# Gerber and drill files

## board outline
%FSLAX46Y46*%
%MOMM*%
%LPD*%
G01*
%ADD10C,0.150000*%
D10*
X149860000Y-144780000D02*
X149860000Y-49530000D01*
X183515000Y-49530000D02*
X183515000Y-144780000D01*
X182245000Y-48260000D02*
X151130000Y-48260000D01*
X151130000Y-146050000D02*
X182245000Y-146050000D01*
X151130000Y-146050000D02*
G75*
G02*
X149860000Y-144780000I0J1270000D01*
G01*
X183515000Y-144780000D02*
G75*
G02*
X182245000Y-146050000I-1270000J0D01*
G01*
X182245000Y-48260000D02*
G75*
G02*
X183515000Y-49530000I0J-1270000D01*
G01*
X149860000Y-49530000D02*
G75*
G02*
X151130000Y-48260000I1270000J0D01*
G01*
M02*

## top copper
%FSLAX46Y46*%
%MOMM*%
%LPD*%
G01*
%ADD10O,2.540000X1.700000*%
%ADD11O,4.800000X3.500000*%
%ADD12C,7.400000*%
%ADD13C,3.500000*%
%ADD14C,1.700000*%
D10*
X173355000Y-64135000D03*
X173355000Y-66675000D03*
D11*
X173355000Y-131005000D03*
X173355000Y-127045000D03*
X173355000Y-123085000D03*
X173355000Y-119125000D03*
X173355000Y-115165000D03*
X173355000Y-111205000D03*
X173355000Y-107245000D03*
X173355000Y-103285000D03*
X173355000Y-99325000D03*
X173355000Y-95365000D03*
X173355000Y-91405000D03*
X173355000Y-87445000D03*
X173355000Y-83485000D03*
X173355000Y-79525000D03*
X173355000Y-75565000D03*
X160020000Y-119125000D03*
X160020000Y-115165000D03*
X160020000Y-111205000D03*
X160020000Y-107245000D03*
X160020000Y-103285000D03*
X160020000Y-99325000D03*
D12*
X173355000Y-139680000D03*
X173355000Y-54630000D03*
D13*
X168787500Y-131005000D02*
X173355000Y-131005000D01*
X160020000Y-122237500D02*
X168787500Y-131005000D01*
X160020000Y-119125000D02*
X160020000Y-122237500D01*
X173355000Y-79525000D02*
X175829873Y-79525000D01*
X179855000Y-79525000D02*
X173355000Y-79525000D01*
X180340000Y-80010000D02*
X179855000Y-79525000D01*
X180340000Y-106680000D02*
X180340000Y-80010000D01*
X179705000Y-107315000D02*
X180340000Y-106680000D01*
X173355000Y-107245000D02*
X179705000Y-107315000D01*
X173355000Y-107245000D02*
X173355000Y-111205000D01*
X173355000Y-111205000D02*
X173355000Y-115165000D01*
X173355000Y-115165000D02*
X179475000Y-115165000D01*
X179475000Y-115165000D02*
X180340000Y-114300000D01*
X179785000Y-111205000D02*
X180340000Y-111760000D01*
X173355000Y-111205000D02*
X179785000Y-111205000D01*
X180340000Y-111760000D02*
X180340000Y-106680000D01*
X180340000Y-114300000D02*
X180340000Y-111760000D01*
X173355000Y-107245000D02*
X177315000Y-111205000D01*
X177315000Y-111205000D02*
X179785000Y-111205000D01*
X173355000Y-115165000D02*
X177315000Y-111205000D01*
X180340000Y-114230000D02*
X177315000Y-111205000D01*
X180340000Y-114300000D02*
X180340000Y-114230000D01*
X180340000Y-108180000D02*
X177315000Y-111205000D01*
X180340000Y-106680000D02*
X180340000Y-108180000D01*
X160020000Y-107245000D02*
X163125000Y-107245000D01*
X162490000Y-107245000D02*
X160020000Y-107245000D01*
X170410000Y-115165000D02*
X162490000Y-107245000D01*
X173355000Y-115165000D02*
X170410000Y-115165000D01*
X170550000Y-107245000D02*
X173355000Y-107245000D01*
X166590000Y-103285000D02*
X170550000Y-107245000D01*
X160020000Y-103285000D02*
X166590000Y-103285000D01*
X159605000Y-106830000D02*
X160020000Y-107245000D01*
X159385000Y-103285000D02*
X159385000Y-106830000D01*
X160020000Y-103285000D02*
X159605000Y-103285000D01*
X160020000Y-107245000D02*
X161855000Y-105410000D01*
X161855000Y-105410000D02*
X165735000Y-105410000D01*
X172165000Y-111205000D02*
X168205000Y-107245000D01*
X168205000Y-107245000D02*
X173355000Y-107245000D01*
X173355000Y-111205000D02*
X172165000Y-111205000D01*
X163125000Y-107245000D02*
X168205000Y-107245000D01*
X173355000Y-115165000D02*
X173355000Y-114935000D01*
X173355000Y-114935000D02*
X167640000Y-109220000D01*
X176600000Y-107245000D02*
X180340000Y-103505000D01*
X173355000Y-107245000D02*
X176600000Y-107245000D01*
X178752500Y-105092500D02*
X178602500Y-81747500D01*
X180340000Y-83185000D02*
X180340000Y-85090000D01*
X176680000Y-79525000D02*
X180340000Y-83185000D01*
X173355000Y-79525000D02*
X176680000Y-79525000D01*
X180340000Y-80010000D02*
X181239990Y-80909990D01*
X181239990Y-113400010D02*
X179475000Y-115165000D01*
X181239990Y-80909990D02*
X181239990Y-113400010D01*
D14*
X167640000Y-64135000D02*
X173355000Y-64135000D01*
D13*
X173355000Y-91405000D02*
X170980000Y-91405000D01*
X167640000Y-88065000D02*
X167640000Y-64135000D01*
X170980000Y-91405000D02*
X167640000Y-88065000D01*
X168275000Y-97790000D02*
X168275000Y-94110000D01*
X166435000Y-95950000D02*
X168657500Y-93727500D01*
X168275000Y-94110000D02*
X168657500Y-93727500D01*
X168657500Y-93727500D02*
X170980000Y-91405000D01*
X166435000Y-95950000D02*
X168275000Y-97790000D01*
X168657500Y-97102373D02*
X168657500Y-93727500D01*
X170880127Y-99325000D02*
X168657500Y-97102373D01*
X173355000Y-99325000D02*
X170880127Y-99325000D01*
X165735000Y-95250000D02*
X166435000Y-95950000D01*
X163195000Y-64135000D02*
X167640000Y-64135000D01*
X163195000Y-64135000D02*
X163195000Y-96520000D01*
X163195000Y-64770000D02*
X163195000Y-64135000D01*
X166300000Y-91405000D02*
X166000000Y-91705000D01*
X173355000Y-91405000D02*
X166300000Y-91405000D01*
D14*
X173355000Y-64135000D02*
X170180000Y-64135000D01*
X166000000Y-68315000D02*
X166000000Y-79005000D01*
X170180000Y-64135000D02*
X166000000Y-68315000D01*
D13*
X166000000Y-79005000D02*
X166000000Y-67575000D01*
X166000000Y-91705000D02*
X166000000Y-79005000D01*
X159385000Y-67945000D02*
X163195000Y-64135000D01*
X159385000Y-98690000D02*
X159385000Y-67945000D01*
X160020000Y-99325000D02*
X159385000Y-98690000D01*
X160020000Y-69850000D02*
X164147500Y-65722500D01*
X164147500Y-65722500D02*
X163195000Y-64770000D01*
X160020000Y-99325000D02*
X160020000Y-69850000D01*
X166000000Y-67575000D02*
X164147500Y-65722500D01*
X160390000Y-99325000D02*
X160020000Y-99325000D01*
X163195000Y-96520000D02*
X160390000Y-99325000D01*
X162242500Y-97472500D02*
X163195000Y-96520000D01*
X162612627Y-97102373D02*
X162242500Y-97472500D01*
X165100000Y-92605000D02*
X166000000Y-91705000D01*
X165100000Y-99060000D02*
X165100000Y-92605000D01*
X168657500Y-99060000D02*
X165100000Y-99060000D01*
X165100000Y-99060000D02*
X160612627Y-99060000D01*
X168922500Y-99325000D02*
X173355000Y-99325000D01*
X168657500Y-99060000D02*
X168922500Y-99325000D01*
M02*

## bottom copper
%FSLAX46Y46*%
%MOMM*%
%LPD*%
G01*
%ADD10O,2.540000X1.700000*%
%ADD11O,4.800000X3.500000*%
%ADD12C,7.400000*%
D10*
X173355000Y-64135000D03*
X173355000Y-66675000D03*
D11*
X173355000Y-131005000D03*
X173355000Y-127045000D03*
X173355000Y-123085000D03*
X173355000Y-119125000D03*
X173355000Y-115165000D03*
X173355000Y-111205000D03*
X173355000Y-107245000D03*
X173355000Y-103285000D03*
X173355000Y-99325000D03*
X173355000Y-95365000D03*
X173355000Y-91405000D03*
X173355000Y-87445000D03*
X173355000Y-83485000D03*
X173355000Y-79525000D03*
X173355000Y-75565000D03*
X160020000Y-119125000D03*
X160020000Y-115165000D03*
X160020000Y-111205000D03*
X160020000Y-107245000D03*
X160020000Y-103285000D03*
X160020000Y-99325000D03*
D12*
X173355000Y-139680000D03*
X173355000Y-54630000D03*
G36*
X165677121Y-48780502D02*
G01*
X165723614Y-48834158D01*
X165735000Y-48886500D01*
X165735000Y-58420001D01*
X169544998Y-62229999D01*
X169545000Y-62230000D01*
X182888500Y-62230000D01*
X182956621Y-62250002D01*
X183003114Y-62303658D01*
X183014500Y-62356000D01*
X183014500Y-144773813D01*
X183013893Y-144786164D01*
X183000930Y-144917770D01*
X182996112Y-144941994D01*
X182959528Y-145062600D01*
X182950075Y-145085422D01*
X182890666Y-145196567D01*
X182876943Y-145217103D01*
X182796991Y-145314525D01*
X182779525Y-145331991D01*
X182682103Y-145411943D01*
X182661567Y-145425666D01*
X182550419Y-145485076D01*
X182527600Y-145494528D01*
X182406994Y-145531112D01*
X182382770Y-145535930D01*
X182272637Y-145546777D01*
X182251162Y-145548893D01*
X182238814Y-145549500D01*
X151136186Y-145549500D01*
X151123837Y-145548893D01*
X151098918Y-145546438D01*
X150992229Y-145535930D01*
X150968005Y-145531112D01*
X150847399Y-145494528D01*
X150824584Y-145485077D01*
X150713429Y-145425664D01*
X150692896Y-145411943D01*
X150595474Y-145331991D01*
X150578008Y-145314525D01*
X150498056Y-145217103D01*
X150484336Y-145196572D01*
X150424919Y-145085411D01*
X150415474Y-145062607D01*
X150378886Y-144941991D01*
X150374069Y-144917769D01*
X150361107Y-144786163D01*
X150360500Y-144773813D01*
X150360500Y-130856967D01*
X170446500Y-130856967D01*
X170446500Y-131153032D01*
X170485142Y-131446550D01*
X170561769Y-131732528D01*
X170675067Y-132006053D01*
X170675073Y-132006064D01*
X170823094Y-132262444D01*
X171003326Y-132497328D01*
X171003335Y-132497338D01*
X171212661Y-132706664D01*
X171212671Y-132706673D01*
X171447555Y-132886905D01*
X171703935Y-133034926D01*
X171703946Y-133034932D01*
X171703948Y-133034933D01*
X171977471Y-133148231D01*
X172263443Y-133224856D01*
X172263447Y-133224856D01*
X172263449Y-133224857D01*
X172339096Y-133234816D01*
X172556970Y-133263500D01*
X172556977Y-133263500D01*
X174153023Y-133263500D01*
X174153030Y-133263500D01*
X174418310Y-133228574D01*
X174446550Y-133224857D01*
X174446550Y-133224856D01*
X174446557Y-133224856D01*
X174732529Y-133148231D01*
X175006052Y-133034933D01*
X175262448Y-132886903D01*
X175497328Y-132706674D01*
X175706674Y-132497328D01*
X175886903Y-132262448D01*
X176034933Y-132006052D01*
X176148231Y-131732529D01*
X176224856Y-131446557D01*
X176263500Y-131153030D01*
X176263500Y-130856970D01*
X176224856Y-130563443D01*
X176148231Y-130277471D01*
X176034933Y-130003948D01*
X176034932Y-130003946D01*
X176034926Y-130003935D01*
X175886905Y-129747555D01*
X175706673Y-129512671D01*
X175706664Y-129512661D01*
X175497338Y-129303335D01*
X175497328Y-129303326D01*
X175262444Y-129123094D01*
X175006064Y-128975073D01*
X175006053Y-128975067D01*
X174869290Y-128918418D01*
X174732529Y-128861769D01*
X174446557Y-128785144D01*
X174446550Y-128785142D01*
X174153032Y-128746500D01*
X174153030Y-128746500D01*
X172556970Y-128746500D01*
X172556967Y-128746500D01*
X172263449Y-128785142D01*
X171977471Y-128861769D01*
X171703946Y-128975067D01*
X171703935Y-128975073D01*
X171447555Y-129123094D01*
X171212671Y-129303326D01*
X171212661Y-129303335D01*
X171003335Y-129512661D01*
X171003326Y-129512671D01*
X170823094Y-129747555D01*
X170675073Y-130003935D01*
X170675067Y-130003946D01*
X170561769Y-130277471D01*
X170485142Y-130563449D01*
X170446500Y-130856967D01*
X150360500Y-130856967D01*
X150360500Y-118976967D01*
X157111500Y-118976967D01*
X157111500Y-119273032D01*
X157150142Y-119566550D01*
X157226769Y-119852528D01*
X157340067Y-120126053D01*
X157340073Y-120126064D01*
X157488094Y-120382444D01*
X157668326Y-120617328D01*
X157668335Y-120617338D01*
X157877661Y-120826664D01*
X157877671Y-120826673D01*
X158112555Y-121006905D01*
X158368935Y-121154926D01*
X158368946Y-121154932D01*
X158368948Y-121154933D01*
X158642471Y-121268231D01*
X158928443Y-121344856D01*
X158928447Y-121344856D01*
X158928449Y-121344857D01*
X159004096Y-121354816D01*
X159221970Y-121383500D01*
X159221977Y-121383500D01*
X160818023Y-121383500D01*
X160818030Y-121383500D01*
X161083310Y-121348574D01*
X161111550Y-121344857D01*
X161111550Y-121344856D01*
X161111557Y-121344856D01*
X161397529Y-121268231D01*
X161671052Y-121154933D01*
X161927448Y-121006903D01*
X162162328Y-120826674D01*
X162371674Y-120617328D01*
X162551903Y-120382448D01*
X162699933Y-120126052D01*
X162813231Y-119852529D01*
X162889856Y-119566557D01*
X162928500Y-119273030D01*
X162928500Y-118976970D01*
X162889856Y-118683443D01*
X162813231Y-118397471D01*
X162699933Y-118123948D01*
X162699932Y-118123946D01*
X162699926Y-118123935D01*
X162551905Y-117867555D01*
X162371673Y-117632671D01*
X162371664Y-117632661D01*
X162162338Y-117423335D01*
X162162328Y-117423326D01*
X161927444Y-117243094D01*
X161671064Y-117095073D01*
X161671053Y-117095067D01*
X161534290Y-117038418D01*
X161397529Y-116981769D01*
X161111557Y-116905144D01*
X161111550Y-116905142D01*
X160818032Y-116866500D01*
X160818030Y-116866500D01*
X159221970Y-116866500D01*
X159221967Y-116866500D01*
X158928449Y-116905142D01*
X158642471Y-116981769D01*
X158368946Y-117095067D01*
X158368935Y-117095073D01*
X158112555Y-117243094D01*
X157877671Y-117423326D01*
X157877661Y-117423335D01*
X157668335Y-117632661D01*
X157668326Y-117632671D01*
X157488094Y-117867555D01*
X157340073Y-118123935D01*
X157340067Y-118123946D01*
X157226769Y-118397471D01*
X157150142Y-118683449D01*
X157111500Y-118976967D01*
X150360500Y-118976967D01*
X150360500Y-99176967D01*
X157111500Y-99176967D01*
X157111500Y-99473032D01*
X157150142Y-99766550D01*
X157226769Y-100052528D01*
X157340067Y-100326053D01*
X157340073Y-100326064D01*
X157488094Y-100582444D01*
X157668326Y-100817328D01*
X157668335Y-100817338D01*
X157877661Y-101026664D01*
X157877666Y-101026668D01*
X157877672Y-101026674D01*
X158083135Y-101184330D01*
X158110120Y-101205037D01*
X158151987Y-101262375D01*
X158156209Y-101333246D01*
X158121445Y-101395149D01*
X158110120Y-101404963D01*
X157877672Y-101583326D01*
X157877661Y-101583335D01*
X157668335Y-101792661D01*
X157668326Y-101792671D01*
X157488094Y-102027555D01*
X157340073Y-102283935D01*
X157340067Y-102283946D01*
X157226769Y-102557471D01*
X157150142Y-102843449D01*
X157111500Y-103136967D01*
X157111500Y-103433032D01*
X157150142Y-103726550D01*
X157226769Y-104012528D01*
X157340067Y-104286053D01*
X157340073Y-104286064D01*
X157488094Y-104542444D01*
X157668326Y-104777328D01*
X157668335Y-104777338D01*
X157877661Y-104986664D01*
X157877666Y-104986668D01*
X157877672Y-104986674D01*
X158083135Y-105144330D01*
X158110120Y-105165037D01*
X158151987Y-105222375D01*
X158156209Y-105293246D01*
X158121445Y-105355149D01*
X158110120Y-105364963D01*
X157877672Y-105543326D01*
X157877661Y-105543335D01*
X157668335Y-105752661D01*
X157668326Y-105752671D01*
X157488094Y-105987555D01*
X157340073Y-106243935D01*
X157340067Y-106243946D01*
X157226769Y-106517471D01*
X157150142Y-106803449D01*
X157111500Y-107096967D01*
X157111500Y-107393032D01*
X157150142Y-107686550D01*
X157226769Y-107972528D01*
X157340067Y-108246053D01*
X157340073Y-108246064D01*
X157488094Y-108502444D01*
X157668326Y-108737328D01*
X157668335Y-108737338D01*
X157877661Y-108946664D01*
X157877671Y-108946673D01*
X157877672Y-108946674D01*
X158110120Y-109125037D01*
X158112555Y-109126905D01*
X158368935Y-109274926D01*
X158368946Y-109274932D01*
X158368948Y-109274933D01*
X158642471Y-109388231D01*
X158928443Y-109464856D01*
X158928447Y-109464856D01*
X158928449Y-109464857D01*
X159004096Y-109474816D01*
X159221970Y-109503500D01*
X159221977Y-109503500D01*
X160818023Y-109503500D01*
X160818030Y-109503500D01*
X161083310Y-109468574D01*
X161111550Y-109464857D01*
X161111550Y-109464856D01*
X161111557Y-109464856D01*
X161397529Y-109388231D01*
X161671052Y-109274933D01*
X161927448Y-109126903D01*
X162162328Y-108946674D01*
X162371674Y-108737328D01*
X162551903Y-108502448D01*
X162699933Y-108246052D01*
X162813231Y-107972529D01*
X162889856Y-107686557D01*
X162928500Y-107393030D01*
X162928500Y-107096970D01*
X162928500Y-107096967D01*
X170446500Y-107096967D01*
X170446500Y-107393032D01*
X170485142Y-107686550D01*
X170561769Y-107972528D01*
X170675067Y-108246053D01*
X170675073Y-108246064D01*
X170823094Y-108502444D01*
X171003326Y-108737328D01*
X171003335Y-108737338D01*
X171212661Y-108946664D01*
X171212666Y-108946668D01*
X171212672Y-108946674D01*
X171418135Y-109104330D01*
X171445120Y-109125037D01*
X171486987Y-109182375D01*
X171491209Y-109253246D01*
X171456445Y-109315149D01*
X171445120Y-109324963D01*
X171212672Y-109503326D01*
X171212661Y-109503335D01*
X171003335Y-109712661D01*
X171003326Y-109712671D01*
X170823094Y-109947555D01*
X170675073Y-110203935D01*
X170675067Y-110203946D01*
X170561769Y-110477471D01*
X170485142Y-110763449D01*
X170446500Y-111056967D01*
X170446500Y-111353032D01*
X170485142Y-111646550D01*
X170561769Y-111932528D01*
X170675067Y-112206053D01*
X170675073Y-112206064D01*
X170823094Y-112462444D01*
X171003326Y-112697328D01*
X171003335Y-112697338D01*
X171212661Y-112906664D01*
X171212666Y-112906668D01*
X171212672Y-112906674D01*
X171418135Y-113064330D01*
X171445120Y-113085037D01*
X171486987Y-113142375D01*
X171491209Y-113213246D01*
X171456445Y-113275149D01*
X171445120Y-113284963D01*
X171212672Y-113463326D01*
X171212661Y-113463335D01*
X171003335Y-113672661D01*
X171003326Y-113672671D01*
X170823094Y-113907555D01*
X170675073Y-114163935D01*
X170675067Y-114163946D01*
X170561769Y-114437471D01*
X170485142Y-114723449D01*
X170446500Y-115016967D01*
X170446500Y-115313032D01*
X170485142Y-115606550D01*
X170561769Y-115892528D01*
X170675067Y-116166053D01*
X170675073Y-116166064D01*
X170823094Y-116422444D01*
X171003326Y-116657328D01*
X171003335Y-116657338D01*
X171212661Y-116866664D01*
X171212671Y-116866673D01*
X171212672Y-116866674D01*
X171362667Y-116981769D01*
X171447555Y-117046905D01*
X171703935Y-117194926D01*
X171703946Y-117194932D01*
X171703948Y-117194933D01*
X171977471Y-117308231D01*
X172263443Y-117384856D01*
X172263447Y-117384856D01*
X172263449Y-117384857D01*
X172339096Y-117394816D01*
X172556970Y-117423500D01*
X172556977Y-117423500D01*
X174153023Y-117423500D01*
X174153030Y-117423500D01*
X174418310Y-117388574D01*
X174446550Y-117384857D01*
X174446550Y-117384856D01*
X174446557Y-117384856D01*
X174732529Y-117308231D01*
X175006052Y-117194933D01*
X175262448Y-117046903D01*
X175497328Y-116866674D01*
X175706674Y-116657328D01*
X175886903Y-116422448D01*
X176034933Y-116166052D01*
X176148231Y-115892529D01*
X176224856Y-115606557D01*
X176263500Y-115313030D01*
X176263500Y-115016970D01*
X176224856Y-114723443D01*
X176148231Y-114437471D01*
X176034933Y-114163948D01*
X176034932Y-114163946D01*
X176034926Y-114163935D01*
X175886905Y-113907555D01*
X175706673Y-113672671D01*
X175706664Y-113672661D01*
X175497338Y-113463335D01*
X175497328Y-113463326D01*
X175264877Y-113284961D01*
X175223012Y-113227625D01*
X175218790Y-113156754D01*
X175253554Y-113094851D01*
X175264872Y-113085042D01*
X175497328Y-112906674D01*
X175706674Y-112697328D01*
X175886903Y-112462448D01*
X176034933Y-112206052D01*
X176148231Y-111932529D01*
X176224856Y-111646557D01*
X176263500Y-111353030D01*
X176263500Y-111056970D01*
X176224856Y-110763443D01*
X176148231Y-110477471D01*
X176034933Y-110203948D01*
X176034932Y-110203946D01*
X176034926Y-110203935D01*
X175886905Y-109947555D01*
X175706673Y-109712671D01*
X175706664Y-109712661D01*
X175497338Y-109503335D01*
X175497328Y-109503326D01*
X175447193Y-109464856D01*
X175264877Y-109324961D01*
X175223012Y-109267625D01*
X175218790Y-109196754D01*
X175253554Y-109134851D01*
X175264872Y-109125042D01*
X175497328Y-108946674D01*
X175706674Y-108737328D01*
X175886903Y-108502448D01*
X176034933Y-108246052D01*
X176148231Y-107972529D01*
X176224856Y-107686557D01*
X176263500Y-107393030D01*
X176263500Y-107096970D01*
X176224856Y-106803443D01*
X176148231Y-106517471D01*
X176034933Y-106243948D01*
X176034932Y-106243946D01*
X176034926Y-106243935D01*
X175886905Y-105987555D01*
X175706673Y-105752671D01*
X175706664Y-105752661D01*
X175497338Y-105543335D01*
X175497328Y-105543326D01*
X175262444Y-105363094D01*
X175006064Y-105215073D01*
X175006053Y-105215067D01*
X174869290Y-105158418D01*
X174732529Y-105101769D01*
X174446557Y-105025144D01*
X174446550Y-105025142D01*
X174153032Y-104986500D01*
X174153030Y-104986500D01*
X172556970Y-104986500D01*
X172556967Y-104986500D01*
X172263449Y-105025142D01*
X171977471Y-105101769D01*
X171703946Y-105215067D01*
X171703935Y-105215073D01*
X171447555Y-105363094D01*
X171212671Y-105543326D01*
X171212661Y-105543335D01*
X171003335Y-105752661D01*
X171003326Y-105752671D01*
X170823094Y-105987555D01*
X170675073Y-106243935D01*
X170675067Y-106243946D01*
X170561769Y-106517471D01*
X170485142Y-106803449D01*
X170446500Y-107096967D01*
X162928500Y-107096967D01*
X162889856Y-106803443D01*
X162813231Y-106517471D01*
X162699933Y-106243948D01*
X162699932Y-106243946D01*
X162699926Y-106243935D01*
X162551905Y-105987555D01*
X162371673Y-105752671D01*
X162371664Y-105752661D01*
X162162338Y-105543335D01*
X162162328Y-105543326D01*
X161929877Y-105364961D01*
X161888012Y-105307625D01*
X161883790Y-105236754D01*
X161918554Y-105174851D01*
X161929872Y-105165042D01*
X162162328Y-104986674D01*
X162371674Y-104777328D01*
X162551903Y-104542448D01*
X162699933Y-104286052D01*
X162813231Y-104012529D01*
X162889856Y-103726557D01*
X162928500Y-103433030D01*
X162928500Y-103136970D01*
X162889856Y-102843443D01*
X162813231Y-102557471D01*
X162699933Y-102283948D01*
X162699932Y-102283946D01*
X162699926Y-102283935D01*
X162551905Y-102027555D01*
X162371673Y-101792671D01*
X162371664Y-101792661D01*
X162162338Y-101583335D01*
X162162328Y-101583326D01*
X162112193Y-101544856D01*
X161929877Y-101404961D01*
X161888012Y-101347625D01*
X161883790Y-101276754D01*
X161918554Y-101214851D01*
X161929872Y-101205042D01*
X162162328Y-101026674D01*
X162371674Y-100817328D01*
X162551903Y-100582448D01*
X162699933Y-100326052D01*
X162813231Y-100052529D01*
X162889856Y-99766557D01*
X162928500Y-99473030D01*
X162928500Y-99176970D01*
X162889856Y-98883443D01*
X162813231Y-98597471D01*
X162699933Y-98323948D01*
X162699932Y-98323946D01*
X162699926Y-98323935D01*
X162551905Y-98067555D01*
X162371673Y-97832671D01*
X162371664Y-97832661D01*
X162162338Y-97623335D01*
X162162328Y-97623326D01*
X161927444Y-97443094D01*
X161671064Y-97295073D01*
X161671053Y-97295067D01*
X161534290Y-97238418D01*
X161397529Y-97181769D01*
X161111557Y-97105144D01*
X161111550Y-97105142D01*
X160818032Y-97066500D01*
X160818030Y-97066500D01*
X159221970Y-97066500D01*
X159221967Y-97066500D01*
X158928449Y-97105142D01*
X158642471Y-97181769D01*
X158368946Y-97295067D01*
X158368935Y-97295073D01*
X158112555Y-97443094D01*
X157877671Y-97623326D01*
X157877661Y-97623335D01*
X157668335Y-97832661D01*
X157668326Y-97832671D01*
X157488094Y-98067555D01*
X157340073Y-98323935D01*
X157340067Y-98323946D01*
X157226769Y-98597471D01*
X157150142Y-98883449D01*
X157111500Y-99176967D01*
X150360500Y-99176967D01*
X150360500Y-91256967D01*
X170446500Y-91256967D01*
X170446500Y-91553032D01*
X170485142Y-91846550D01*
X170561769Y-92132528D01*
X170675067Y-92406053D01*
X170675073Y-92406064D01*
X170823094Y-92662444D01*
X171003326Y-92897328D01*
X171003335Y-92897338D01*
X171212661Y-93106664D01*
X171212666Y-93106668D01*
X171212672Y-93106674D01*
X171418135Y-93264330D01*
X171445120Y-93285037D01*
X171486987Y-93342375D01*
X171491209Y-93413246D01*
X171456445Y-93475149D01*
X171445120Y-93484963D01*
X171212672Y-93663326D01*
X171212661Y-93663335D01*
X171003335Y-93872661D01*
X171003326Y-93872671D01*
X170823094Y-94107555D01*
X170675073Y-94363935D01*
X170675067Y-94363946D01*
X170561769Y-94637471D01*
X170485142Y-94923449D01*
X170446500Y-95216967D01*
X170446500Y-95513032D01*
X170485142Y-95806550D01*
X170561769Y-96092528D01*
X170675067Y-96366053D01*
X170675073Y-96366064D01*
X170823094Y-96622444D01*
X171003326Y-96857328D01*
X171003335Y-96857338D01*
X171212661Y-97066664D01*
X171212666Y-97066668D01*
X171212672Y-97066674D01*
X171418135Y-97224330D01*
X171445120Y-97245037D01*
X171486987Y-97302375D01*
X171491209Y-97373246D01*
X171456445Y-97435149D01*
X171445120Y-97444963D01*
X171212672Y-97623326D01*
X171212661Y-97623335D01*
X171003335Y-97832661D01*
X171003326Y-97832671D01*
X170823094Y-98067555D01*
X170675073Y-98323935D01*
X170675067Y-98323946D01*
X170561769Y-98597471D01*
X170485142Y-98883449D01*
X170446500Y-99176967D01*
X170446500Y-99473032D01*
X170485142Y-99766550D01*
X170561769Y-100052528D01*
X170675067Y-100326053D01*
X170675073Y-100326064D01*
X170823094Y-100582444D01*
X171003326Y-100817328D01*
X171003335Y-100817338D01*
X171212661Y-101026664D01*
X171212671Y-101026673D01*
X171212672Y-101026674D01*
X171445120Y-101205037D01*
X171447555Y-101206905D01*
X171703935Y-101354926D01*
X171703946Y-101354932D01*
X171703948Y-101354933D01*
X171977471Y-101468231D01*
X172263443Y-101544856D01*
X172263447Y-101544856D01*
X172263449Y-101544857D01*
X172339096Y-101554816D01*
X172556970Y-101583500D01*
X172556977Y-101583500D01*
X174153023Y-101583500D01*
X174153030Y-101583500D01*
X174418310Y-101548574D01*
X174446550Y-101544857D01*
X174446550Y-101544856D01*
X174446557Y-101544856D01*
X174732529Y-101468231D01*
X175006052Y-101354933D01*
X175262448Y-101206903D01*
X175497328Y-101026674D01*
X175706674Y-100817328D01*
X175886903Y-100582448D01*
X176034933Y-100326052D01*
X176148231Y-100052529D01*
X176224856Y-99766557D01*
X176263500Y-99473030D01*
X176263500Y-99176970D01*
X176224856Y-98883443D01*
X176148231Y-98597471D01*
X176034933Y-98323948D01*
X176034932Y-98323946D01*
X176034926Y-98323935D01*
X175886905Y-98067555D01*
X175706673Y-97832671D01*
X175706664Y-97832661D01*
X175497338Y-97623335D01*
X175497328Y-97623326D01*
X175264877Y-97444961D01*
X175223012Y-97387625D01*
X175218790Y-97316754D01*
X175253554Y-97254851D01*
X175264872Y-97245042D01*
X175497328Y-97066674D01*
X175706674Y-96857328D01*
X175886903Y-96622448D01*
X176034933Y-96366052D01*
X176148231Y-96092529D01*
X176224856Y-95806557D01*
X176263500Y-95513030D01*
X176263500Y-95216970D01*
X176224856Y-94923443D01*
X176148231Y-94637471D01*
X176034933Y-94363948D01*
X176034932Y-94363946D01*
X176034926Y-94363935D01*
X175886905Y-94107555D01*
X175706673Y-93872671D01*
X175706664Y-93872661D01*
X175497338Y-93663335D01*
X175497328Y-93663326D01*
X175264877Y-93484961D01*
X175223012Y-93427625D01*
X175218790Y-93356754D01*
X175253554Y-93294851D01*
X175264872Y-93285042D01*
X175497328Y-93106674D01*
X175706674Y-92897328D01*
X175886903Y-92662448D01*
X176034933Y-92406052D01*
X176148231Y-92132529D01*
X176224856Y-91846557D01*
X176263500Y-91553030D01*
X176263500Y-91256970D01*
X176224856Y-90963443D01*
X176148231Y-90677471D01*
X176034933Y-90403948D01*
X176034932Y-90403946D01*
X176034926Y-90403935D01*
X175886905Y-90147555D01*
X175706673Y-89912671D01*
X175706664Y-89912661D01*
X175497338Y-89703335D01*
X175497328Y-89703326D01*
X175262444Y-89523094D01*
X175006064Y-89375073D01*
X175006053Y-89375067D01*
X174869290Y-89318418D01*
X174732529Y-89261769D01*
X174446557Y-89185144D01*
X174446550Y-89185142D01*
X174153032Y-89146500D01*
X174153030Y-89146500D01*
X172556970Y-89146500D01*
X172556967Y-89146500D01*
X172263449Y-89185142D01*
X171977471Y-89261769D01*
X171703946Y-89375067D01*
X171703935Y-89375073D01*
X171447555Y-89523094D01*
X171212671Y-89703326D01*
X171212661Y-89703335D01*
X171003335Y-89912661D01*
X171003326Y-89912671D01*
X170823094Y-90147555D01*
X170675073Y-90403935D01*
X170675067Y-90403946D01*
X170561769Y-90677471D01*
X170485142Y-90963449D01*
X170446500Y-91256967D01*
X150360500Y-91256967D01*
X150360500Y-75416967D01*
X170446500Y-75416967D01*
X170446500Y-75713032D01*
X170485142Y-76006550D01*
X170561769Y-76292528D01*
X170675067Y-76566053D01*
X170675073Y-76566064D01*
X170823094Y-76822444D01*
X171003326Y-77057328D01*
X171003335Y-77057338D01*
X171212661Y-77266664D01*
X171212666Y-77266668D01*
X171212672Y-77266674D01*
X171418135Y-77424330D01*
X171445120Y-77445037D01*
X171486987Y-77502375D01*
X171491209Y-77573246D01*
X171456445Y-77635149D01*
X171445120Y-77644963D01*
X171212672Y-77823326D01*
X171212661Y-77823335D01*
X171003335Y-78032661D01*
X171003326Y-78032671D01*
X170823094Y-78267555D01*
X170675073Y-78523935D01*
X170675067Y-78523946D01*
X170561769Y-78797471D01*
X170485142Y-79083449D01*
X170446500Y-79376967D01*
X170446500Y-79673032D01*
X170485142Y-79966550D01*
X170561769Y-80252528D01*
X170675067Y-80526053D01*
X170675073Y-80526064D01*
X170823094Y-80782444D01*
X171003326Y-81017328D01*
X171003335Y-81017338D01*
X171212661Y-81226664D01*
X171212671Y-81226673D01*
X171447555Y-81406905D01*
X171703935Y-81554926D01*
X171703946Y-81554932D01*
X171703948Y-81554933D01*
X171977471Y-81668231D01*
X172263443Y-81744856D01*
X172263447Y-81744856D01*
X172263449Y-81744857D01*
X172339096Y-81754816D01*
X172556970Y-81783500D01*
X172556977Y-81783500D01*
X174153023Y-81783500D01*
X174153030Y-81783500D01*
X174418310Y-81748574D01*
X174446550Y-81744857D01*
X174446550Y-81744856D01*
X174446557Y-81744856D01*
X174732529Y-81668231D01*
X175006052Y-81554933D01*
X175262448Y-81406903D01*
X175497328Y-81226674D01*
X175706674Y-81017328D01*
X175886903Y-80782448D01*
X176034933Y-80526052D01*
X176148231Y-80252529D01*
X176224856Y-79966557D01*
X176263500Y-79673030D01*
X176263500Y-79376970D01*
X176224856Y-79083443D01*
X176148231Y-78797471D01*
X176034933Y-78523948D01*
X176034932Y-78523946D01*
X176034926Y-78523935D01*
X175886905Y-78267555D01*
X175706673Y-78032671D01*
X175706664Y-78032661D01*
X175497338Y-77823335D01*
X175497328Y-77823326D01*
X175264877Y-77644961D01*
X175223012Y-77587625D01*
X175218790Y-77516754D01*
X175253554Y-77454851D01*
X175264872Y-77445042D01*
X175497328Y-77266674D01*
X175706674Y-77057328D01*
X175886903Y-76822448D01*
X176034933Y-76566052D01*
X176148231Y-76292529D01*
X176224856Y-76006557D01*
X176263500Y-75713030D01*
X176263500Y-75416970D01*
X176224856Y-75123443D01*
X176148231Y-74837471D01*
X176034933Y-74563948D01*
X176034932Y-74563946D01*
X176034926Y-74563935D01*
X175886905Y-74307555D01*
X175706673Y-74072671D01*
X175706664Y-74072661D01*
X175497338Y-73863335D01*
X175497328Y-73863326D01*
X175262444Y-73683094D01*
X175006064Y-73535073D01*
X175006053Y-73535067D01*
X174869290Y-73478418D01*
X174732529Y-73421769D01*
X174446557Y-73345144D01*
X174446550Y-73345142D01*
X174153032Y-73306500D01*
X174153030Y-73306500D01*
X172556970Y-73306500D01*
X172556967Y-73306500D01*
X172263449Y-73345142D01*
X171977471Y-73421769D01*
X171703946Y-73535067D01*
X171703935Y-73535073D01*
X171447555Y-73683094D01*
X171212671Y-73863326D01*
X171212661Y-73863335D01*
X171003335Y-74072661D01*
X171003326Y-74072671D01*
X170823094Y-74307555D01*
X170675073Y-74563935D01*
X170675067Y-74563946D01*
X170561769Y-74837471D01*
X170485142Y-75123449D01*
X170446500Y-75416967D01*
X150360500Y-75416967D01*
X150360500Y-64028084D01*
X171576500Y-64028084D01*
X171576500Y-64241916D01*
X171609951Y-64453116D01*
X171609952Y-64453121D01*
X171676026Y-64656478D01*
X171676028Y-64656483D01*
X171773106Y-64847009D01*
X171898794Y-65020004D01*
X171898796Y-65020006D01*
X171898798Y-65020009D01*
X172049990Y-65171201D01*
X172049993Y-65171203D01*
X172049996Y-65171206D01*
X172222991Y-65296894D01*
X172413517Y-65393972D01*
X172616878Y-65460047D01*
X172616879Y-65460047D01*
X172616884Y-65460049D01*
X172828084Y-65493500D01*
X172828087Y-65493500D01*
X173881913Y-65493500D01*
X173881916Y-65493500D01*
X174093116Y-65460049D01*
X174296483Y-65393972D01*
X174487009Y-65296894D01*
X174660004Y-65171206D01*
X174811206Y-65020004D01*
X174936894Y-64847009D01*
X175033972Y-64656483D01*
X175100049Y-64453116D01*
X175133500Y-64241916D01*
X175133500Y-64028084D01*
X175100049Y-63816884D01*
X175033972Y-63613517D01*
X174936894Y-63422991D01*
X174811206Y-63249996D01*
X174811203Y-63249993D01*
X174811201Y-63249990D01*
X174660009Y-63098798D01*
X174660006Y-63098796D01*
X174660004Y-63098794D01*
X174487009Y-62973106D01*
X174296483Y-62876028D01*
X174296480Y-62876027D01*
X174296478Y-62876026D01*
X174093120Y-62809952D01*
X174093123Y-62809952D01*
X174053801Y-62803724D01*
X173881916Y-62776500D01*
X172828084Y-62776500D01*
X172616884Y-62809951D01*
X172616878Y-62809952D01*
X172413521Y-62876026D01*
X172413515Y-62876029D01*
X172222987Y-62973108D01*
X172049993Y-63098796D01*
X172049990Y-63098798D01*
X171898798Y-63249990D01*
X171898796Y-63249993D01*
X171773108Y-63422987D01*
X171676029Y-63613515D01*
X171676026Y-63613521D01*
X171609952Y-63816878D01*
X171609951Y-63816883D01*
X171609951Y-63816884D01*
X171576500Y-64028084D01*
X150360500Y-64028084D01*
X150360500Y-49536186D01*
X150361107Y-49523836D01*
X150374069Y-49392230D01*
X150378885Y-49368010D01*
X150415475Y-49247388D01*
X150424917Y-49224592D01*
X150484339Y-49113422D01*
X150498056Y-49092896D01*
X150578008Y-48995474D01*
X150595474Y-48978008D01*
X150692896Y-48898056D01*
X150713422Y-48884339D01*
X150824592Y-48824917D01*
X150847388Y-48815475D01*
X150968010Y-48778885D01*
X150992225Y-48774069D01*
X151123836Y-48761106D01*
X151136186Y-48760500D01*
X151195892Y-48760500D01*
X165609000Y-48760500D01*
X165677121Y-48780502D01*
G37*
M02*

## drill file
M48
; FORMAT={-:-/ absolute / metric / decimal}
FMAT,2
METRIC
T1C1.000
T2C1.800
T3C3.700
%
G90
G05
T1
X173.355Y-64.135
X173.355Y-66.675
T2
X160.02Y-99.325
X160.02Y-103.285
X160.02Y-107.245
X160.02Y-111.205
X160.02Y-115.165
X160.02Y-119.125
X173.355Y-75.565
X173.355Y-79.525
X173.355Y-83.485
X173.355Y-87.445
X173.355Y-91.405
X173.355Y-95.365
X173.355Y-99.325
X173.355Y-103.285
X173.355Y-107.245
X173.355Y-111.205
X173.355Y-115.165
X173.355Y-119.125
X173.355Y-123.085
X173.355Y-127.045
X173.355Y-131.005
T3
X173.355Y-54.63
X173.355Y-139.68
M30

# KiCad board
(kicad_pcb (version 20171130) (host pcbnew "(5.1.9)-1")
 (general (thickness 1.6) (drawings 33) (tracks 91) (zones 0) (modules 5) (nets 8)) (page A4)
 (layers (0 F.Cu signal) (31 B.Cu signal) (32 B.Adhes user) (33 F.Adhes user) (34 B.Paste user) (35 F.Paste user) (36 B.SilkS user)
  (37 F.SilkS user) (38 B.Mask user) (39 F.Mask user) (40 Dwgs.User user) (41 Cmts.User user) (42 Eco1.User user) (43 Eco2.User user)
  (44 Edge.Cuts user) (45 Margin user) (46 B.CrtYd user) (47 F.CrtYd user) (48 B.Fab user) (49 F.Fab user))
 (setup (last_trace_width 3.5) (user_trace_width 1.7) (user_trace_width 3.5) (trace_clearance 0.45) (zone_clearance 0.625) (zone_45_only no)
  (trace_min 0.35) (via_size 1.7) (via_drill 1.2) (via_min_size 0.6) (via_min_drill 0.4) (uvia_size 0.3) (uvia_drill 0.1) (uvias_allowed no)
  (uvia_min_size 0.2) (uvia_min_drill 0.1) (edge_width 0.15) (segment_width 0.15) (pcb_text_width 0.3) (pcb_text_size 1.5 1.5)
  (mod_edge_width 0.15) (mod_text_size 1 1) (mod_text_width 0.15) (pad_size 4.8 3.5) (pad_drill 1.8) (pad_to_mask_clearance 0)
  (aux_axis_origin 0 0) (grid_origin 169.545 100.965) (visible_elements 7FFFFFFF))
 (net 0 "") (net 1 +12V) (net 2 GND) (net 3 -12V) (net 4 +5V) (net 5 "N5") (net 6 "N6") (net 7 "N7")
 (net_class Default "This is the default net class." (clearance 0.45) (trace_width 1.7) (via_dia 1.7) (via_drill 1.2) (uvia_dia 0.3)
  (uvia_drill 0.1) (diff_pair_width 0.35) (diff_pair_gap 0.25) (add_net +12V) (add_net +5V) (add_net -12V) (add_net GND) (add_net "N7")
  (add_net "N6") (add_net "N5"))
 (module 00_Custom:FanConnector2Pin (layer F.Cu) (at 173.355 64.135)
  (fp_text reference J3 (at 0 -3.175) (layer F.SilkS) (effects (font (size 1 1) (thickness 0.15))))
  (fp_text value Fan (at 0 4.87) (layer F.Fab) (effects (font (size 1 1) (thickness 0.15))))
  (pad 1 thru_hole oval (at 0 0) (size 2.54 1.7) (drill 1) (layers *.Cu *.Mask) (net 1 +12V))
  (pad 2 thru_hole oval (at 0 2.54) (size 2.54 1.7) (drill 1) (layers *.Cu *.Mask) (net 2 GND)))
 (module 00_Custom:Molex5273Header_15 (layer F.Cu) (at 173.355 75.565)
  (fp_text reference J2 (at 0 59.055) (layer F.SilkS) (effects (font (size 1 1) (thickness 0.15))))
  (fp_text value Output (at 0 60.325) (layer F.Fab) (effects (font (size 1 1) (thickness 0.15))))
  (pad 15 thru_hole oval (at 0 55.44) (size 4.8 3.5) (drill 1.8) (layers *.Cu *.Mask) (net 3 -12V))
  (pad 14 thru_hole oval (at 0 51.48) (size 4.8 3.5) (drill 1.8) (layers *.Cu *.Mask) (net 2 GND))
  (pad 13 thru_hole oval (at 0 47.52) (size 4.8 3.5) (drill 1.8) (layers *.Cu *.Mask) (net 2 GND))
  (pad 12 thru_hole oval (at 0 43.56) (size 4.8 3.5) (drill 1.8) (layers *.Cu *.Mask) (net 2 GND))
  (pad 11 thru_hole oval (at 0 39.6) (size 4.8 3.5) (drill 1.8) (layers *.Cu *.Mask) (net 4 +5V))
  (pad 10 thru_hole oval (at 0 35.64) (size 4.8 3.5) (drill 1.8) (layers *.Cu *.Mask) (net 4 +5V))
  (pad 9 thru_hole oval (at 0 31.68) (size 4.8 3.5) (drill 1.8) (layers *.Cu *.Mask) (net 4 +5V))
  (pad 8 thru_hole oval (at 0 27.72) (size 4.8 3.5) (drill 1.8) (layers *.Cu *.Mask) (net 2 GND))
  (pad 7 thru_hole oval (at 0 23.76) (size 4.8 3.5) (drill 1.8) (layers *.Cu *.Mask) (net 1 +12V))
  (pad 6 thru_hole oval (at 0 19.8) (size 4.8 3.5) (drill 1.8) (layers *.Cu *.Mask) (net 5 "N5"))
  (pad 5 thru_hole oval (at 0 15.84) (size 4.8 3.5) (drill 1.8) (layers *.Cu *.Mask) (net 1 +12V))
  (pad 4 thru_hole oval (at 0 11.88) (size 4.8 3.5) (drill 1.8) (layers *.Cu *.Mask) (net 2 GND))
  (pad 3 thru_hole oval (at 0 7.92) (size 4.8 3.5) (drill 1.8) (layers *.Cu *.Mask) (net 2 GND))
  (pad 2 thru_hole oval (at 0 3.96) (size 4.8 3.5) (drill 1.8) (layers *.Cu *.Mask) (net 4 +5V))
  (pad 1 thru_hole oval (at 0 0) (size 4.8 3.5) (drill 1.8) (layers *.Cu *.Mask) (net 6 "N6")))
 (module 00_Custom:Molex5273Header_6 (layer F.Cu) (at 160.02 99.325)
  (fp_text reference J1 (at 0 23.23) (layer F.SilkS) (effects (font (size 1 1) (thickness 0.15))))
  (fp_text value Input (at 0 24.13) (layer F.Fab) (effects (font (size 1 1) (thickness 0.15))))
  (pad 6 thru_hole oval (at 0 19.8) (size 4.8 3.5) (drill 1.8) (layers *.Cu *.Mask) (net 3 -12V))
  (pad 5 thru_hole oval (at 0 15.84) (size 4.8 3.5) (drill 1.8) (layers *.Cu *.Mask) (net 2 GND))
  (pad 4 thru_hole oval (at 0 11.88) (size 4.8 3.5) (drill 1.8) (layers *.Cu *.Mask) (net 2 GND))
  (pad 3 thru_hole oval (at 0 7.92) (size 4.8 3.5) (drill 1.8) (layers *.Cu *.Mask) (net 4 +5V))
  (pad 2 thru_hole oval (at 0 3.96) (size 4.8 3.5) (drill 1.8) (layers *.Cu *.Mask) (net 4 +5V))
  (pad 1 thru_hole oval (at 0 0) (size 4.8 3.5) (drill 1.8) (layers *.Cu *.Mask) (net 1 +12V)))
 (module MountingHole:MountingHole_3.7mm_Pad (layer F.Cu) (at 173.355 139.68)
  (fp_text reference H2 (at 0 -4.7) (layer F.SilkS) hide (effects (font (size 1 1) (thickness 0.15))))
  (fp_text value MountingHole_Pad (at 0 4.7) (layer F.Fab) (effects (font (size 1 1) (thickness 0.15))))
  (pad 1 thru_hole circle (at 0 0) (size 7.4 7.4) (drill 3.7) (layers *.Cu *.Mask) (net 2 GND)))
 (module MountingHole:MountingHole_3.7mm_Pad (layer F.Cu) (at 173.355 54.63)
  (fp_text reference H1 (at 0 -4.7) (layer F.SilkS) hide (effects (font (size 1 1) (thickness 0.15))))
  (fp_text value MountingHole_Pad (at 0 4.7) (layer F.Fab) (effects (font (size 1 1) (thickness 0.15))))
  (pad 1 thru_hole circle (at 0 0) (size 7.4 7.4) (drill 3.7) (layers *.Cu *.Mask) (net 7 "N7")))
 (gr_line (start 149.86 144.78) (end 149.86 49.53) (layer Edge.Cuts) (width 0.15))
 (gr_line (start 183.515 49.53) (end 183.515 144.78) (layer Edge.Cuts) (width 0.15))
 (gr_line (start 182.245 48.26) (end 151.13 48.26) (layer Edge.Cuts) (width 0.15))
 (gr_line (start 151.13 146.05) (end 182.245 146.05) (layer Edge.Cuts) (width 0.15))
 (gr_arc (start 151.13 144.78) (end 149.86 144.78) (angle -90) (layer Edge.Cuts) (width 0.15))
 (gr_arc (start 182.245 144.78) (end 182.245 146.05) (angle -90) (layer Edge.Cuts) (width 0.15))
 (gr_arc (start 182.245 49.53) (end 183.515 49.53) (angle -90) (layer Edge.Cuts) (width 0.15))
 (gr_arc (start 151.13 49.53) (end 151.13 48.26) (angle -90) (layer Edge.Cuts) (width 0.15))
 (segment (start 168.7875 131.005) (end 173.355 131.005) (width 3.5) (layer F.Cu) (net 3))
 (segment (start 160.02 122.2375) (end 168.7875 131.005) (width 3.5) (layer F.Cu) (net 3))
 (segment (start 160.02 119.125) (end 160.02 122.2375) (width 3.5) (layer F.Cu) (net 3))
 (segment (start 173.355 79.525) (end 175.829873 79.525) (width 3.5) (layer F.Cu) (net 4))
 (segment (start 179.855 79.525) (end 173.355 79.525) (width 3.5) (layer F.Cu) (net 4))
 (segment (start 180.34 80.01) (end 179.855 79.525) (width 3.5) (layer F.Cu) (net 4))
 (segment (start 180.34 106.68) (end 180.34 80.01) (width 3.5) (layer F.Cu) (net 4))
 (segment (start 179.705 107.315) (end 180.34 106.68) (width 3.5) (layer F.Cu) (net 4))
 (segment (start 173.355 107.245) (end 179.705 107.315) (width 3.5) (layer F.Cu) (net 4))
 (segment (start 173.355 107.245) (end 173.355 111.205) (width 3.5) (layer F.Cu) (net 4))
 (segment (start 173.355 111.205) (end 173.355 115.165) (width 3.5) (layer F.Cu) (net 4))
 (segment (start 173.355 115.165) (end 179.475 115.165) (width 3.5) (layer F.Cu) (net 4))
 (segment (start 179.475 115.165) (end 180.34 114.3) (width 3.5) (layer F.Cu) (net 4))
 (segment (start 179.785 111.205) (end 180.34 111.76) (width 3.5) (layer F.Cu) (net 4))
 (segment (start 173.355 111.205) (end 179.785 111.205) (width 3.5) (layer F.Cu) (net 4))
 (segment (start 180.34 111.76) (end 180.34 106.68) (width 3.5) (layer F.Cu) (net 4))
 (segment (start 180.34 114.3) (end 180.34 111.76) (width 3.5) (layer F.Cu) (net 4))
 (segment (start 173.355 107.245) (end 177.315 111.205) (width 3.5) (layer F.Cu) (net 4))
 (segment (start 177.315 111.205) (end 179.785 111.205) (width 3.5) (layer F.Cu) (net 4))
 (segment (start 173.355 115.165) (end 177.315 111.205) (width 3.5) (layer F.Cu) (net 4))
 (segment (start 180.34 114.23) (end 177.315 111.205) (width 3.5) (layer F.Cu) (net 4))
 (segment (start 180.34 114.3) (end 180.34 114.23) (width 3.5) (layer F.Cu) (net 4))
 (segment (start 180.34 108.18) (end 177.315 111.205) (width 3.5) (layer F.Cu) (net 4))
 (segment (start 180.34 106.68) (end 180.34 108.18) (width 3.5) (layer F.Cu) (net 4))
 (segment (start 160.02 107.245) (end 163.125 107.245) (width 3.5) (layer F.Cu) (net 4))
 (segment (start 162.49 107.245) (end 160.02 107.245) (width 3.5) (layer F.Cu) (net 4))
 (segment (start 170.41 115.165) (end 162.49 107.245) (width 3.5) (layer F.Cu) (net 4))
 (segment (start 173.355 115.165) (end 170.41 115.165) (width 3.5) (layer F.Cu) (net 4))
 (segment (start 170.55 107.245) (end 173.355 107.245) (width 3.5) (layer F.Cu) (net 4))
 (segment (start 166.59 103.285) (end 170.55 107.245) (width 3.5) (layer F.Cu) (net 4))
 (segment (start 160.02 103.285) (end 166.59 103.285) (width 3.5) (layer F.Cu) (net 4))
 (segment (start 159.605 106.83) (end 160.02 107.245) (width 3.5) (layer F.Cu) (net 4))
 (segment (start 159.385 103.285) (end 159.385 106.83) (width 3.5) (layer F.Cu) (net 4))
 (segment (start 160.02 103.285) (end 159.605 103.285) (width 3.5) (layer F.Cu) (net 4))
 (segment (start 160.02 107.245) (end 161.855 105.41) (width 3.5) (layer F.Cu) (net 4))
 (segment (start 161.855 105.41) (end 165.735 105.41) (width 3.5) (layer F.Cu) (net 4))
 (segment (start 172.165 111.205) (end 168.205 107.245) (width 3.5) (layer F.Cu) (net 4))
 (segment (start 168.205 107.245) (end 173.355 107.245) (width 3.5) (layer F.Cu) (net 4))
 (segment (start 173.355 111.205) (end 172.165 111.205) (width 3.5) (layer F.Cu) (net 4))
 (segment (start 163.125 107.245) (end 168.205 107.245) (width 3.5) (layer F.Cu) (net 4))
 (segment (start 173.355 115.165) (end 173.355 114.935) (width 3.5) (layer F.Cu) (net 4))
 (segment (start 173.355 114.935) (end 167.64 109.22) (width 3.5) (layer F.Cu) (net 4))
 (segment (start 176.6 107.245) (end 180.34 103.505) (width 3.5) (layer F.Cu) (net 4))
 (segment (start 173.355 107.245) (end 176.6 107.245) (width 3.5) (layer F.Cu) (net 4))
 (segment (start 178.7525 105.0925) (end 178.6025 81.7475) (width 3.5) (layer F.Cu) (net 4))
 (segment (start 180.34 83.185) (end 180.34 85.09) (width 3.5) (layer F.Cu) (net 4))
 (segment (start 176.68 79.525) (end 180.34 83.185) (width 3.5) (layer F.Cu) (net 4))
 (segment (start 173.355 79.525) (end 176.68 79.525) (width 3.5) (layer F.Cu) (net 4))
 (segment (start 180.34 80.01) (end 181.23999 80.90999) (width 3.5) (layer F.Cu) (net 4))
 (segment (start 181.23999 113.40001) (end 179.475 115.165) (width 3.5) (layer F.Cu) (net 4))
 (segment (start 181.23999 80.90999) (end 181.23999 113.40001) (width 3.5) (layer F.Cu) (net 4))
 (segment (start 167.64 64.135) (end 173.355 64.135) (width 1.7) (layer F.Cu) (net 1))
 (segment (start 173.355 91.405) (end 170.98 91.405) (width 3.5) (layer F.Cu) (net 1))
 (segment (start 167.64 88.065) (end 167.64 64.135) (width 3.5) (layer F.Cu) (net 1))
 (segment (start 170.98 91.405) (end 167.64 88.065) (width 3.5) (layer F.Cu) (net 1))
 (segment (start 168.275 97.79) (end 168.275 94.11) (width 3.5) (layer F.Cu) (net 1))
 (segment (start 166.435 95.95) (end 168.6575 93.7275) (width 3.5) (layer F.Cu) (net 1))
 (segment (start 168.275 94.11) (end 168.6575 93.7275) (width 3.5) (layer F.Cu) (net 1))
 (segment (start 168.6575 93.7275) (end 170.98 91.405) (width 3.5) (layer F.Cu) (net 1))
 (segment (start 166.435 95.95) (end 168.275 97.79) (width 3.5) (layer F.Cu) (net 1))
 (segment (start 168.6575 97.102373) (end 168.6575 93.7275) (width 3.5) (layer F.Cu) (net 1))
 (segment (start 170.880127 99.325) (end 168.6575 97.102373) (width 3.5) (layer F.Cu) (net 1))
 (segment (start 173.355 99.325) (end 170.880127 99.325) (width 3.5) (layer F.Cu) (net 1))
 (segment (start 165.735 95.25) (end 166.435 95.95) (width 3.5) (layer F.Cu) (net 1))
 (segment (start 163.195 64.135) (end 167.64 64.135) (width 3.5) (layer F.Cu) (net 1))
 (segment (start 163.195 64.135) (end 163.195 96.52) (width 3.5) (layer F.Cu) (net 1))
 (segment (start 163.195 64.77) (end 163.195 64.135) (width 3.5) (layer F.Cu) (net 1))
 (segment (start 166.3 91.405) (end 166 91.705) (width 3.5) (layer F.Cu) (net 1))
 (segment (start 173.355 91.405) (end 166.3 91.405) (width 3.5) (layer F.Cu) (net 1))
 (segment (start 173.355 64.135) (end 170.18 64.135) (width 1.7) (layer F.Cu) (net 1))
 (segment (start 166 68.315) (end 166 79.005) (width 1.7) (layer F.Cu) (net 1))
 (segment (start 170.18 64.135) (end 166 68.315) (width 1.7) (layer F.Cu) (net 1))
 (segment (start 166 79.005) (end 166 67.575) (width 3.5) (layer F.Cu) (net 1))
 (segment (start 166 91.705) (end 166 79.005) (width 3.5) (layer F.Cu) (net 1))
 (segment (start 159.385 67.945) (end 163.195 64.135) (width 3.5) (layer F.Cu) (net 1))
 (segment (start 159.385 98.69) (end 159.385 67.945) (width 3.5) (layer F.Cu) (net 1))
 (segment (start 160.02 99.325) (end 159.385 98.69) (width 3.5) (layer F.Cu) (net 1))
 (segment (start 160.02 69.85) (end 164.1475 65.7225) (width 3.5) (layer F.Cu) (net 1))
 (segment (start 164.1475 65.7225) (end 163.195 64.77) (width 3.5) (layer F.Cu) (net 1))
 (segment (start 160.02 99.325) (end 160.02 69.85) (width 3.5) (layer F.Cu) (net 1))
 (segment (start 166 67.575) (end 164.1475 65.7225) (width 3.5) (layer F.Cu) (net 1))
 (segment (start 160.39 99.325) (end 160.02 99.325) (width 3.5) (layer F.Cu) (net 1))
 (segment (start 163.195 96.52) (end 160.39 99.325) (width 3.5) (layer F.Cu) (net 1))
 (segment (start 162.2425 97.4725) (end 163.195 96.52) (width 3.5) (layer F.Cu) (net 1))
 (segment (start 162.612627 97.102373) (end 162.2425 97.4725) (width 3.5) (layer F.Cu) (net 1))
 (segment (start 165.1 92.605) (end 166 91.705) (width 3.5) (layer F.Cu) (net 1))
 (segment (start 165.1 99.06) (end 165.1 92.605) (width 3.5) (layer F.Cu) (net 1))
 (segment (start 168.6575 99.06) (end 165.1 99.06) (width 3.5) (layer F.Cu) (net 1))
 (segment (start 165.1 99.06) (end 160.612627 99.06) (width 3.5) (layer F.Cu) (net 1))
 (segment (start 168.9225 99.325) (end 173.355 99.325) (width 3.5) (layer F.Cu) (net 1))
 (segment (start 168.6575 99.06) (end 168.9225 99.325) (width 3.5) (layer F.Cu) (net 1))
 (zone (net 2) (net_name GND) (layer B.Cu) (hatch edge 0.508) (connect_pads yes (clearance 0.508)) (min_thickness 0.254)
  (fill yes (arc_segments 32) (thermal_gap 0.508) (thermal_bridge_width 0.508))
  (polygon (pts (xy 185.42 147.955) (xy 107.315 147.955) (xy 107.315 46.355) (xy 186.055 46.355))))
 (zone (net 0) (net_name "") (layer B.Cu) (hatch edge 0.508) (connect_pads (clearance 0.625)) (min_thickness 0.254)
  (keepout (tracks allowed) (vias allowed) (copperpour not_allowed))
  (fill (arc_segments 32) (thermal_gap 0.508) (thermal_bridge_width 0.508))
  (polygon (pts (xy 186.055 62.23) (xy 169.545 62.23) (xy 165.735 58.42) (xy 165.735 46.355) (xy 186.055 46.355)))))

